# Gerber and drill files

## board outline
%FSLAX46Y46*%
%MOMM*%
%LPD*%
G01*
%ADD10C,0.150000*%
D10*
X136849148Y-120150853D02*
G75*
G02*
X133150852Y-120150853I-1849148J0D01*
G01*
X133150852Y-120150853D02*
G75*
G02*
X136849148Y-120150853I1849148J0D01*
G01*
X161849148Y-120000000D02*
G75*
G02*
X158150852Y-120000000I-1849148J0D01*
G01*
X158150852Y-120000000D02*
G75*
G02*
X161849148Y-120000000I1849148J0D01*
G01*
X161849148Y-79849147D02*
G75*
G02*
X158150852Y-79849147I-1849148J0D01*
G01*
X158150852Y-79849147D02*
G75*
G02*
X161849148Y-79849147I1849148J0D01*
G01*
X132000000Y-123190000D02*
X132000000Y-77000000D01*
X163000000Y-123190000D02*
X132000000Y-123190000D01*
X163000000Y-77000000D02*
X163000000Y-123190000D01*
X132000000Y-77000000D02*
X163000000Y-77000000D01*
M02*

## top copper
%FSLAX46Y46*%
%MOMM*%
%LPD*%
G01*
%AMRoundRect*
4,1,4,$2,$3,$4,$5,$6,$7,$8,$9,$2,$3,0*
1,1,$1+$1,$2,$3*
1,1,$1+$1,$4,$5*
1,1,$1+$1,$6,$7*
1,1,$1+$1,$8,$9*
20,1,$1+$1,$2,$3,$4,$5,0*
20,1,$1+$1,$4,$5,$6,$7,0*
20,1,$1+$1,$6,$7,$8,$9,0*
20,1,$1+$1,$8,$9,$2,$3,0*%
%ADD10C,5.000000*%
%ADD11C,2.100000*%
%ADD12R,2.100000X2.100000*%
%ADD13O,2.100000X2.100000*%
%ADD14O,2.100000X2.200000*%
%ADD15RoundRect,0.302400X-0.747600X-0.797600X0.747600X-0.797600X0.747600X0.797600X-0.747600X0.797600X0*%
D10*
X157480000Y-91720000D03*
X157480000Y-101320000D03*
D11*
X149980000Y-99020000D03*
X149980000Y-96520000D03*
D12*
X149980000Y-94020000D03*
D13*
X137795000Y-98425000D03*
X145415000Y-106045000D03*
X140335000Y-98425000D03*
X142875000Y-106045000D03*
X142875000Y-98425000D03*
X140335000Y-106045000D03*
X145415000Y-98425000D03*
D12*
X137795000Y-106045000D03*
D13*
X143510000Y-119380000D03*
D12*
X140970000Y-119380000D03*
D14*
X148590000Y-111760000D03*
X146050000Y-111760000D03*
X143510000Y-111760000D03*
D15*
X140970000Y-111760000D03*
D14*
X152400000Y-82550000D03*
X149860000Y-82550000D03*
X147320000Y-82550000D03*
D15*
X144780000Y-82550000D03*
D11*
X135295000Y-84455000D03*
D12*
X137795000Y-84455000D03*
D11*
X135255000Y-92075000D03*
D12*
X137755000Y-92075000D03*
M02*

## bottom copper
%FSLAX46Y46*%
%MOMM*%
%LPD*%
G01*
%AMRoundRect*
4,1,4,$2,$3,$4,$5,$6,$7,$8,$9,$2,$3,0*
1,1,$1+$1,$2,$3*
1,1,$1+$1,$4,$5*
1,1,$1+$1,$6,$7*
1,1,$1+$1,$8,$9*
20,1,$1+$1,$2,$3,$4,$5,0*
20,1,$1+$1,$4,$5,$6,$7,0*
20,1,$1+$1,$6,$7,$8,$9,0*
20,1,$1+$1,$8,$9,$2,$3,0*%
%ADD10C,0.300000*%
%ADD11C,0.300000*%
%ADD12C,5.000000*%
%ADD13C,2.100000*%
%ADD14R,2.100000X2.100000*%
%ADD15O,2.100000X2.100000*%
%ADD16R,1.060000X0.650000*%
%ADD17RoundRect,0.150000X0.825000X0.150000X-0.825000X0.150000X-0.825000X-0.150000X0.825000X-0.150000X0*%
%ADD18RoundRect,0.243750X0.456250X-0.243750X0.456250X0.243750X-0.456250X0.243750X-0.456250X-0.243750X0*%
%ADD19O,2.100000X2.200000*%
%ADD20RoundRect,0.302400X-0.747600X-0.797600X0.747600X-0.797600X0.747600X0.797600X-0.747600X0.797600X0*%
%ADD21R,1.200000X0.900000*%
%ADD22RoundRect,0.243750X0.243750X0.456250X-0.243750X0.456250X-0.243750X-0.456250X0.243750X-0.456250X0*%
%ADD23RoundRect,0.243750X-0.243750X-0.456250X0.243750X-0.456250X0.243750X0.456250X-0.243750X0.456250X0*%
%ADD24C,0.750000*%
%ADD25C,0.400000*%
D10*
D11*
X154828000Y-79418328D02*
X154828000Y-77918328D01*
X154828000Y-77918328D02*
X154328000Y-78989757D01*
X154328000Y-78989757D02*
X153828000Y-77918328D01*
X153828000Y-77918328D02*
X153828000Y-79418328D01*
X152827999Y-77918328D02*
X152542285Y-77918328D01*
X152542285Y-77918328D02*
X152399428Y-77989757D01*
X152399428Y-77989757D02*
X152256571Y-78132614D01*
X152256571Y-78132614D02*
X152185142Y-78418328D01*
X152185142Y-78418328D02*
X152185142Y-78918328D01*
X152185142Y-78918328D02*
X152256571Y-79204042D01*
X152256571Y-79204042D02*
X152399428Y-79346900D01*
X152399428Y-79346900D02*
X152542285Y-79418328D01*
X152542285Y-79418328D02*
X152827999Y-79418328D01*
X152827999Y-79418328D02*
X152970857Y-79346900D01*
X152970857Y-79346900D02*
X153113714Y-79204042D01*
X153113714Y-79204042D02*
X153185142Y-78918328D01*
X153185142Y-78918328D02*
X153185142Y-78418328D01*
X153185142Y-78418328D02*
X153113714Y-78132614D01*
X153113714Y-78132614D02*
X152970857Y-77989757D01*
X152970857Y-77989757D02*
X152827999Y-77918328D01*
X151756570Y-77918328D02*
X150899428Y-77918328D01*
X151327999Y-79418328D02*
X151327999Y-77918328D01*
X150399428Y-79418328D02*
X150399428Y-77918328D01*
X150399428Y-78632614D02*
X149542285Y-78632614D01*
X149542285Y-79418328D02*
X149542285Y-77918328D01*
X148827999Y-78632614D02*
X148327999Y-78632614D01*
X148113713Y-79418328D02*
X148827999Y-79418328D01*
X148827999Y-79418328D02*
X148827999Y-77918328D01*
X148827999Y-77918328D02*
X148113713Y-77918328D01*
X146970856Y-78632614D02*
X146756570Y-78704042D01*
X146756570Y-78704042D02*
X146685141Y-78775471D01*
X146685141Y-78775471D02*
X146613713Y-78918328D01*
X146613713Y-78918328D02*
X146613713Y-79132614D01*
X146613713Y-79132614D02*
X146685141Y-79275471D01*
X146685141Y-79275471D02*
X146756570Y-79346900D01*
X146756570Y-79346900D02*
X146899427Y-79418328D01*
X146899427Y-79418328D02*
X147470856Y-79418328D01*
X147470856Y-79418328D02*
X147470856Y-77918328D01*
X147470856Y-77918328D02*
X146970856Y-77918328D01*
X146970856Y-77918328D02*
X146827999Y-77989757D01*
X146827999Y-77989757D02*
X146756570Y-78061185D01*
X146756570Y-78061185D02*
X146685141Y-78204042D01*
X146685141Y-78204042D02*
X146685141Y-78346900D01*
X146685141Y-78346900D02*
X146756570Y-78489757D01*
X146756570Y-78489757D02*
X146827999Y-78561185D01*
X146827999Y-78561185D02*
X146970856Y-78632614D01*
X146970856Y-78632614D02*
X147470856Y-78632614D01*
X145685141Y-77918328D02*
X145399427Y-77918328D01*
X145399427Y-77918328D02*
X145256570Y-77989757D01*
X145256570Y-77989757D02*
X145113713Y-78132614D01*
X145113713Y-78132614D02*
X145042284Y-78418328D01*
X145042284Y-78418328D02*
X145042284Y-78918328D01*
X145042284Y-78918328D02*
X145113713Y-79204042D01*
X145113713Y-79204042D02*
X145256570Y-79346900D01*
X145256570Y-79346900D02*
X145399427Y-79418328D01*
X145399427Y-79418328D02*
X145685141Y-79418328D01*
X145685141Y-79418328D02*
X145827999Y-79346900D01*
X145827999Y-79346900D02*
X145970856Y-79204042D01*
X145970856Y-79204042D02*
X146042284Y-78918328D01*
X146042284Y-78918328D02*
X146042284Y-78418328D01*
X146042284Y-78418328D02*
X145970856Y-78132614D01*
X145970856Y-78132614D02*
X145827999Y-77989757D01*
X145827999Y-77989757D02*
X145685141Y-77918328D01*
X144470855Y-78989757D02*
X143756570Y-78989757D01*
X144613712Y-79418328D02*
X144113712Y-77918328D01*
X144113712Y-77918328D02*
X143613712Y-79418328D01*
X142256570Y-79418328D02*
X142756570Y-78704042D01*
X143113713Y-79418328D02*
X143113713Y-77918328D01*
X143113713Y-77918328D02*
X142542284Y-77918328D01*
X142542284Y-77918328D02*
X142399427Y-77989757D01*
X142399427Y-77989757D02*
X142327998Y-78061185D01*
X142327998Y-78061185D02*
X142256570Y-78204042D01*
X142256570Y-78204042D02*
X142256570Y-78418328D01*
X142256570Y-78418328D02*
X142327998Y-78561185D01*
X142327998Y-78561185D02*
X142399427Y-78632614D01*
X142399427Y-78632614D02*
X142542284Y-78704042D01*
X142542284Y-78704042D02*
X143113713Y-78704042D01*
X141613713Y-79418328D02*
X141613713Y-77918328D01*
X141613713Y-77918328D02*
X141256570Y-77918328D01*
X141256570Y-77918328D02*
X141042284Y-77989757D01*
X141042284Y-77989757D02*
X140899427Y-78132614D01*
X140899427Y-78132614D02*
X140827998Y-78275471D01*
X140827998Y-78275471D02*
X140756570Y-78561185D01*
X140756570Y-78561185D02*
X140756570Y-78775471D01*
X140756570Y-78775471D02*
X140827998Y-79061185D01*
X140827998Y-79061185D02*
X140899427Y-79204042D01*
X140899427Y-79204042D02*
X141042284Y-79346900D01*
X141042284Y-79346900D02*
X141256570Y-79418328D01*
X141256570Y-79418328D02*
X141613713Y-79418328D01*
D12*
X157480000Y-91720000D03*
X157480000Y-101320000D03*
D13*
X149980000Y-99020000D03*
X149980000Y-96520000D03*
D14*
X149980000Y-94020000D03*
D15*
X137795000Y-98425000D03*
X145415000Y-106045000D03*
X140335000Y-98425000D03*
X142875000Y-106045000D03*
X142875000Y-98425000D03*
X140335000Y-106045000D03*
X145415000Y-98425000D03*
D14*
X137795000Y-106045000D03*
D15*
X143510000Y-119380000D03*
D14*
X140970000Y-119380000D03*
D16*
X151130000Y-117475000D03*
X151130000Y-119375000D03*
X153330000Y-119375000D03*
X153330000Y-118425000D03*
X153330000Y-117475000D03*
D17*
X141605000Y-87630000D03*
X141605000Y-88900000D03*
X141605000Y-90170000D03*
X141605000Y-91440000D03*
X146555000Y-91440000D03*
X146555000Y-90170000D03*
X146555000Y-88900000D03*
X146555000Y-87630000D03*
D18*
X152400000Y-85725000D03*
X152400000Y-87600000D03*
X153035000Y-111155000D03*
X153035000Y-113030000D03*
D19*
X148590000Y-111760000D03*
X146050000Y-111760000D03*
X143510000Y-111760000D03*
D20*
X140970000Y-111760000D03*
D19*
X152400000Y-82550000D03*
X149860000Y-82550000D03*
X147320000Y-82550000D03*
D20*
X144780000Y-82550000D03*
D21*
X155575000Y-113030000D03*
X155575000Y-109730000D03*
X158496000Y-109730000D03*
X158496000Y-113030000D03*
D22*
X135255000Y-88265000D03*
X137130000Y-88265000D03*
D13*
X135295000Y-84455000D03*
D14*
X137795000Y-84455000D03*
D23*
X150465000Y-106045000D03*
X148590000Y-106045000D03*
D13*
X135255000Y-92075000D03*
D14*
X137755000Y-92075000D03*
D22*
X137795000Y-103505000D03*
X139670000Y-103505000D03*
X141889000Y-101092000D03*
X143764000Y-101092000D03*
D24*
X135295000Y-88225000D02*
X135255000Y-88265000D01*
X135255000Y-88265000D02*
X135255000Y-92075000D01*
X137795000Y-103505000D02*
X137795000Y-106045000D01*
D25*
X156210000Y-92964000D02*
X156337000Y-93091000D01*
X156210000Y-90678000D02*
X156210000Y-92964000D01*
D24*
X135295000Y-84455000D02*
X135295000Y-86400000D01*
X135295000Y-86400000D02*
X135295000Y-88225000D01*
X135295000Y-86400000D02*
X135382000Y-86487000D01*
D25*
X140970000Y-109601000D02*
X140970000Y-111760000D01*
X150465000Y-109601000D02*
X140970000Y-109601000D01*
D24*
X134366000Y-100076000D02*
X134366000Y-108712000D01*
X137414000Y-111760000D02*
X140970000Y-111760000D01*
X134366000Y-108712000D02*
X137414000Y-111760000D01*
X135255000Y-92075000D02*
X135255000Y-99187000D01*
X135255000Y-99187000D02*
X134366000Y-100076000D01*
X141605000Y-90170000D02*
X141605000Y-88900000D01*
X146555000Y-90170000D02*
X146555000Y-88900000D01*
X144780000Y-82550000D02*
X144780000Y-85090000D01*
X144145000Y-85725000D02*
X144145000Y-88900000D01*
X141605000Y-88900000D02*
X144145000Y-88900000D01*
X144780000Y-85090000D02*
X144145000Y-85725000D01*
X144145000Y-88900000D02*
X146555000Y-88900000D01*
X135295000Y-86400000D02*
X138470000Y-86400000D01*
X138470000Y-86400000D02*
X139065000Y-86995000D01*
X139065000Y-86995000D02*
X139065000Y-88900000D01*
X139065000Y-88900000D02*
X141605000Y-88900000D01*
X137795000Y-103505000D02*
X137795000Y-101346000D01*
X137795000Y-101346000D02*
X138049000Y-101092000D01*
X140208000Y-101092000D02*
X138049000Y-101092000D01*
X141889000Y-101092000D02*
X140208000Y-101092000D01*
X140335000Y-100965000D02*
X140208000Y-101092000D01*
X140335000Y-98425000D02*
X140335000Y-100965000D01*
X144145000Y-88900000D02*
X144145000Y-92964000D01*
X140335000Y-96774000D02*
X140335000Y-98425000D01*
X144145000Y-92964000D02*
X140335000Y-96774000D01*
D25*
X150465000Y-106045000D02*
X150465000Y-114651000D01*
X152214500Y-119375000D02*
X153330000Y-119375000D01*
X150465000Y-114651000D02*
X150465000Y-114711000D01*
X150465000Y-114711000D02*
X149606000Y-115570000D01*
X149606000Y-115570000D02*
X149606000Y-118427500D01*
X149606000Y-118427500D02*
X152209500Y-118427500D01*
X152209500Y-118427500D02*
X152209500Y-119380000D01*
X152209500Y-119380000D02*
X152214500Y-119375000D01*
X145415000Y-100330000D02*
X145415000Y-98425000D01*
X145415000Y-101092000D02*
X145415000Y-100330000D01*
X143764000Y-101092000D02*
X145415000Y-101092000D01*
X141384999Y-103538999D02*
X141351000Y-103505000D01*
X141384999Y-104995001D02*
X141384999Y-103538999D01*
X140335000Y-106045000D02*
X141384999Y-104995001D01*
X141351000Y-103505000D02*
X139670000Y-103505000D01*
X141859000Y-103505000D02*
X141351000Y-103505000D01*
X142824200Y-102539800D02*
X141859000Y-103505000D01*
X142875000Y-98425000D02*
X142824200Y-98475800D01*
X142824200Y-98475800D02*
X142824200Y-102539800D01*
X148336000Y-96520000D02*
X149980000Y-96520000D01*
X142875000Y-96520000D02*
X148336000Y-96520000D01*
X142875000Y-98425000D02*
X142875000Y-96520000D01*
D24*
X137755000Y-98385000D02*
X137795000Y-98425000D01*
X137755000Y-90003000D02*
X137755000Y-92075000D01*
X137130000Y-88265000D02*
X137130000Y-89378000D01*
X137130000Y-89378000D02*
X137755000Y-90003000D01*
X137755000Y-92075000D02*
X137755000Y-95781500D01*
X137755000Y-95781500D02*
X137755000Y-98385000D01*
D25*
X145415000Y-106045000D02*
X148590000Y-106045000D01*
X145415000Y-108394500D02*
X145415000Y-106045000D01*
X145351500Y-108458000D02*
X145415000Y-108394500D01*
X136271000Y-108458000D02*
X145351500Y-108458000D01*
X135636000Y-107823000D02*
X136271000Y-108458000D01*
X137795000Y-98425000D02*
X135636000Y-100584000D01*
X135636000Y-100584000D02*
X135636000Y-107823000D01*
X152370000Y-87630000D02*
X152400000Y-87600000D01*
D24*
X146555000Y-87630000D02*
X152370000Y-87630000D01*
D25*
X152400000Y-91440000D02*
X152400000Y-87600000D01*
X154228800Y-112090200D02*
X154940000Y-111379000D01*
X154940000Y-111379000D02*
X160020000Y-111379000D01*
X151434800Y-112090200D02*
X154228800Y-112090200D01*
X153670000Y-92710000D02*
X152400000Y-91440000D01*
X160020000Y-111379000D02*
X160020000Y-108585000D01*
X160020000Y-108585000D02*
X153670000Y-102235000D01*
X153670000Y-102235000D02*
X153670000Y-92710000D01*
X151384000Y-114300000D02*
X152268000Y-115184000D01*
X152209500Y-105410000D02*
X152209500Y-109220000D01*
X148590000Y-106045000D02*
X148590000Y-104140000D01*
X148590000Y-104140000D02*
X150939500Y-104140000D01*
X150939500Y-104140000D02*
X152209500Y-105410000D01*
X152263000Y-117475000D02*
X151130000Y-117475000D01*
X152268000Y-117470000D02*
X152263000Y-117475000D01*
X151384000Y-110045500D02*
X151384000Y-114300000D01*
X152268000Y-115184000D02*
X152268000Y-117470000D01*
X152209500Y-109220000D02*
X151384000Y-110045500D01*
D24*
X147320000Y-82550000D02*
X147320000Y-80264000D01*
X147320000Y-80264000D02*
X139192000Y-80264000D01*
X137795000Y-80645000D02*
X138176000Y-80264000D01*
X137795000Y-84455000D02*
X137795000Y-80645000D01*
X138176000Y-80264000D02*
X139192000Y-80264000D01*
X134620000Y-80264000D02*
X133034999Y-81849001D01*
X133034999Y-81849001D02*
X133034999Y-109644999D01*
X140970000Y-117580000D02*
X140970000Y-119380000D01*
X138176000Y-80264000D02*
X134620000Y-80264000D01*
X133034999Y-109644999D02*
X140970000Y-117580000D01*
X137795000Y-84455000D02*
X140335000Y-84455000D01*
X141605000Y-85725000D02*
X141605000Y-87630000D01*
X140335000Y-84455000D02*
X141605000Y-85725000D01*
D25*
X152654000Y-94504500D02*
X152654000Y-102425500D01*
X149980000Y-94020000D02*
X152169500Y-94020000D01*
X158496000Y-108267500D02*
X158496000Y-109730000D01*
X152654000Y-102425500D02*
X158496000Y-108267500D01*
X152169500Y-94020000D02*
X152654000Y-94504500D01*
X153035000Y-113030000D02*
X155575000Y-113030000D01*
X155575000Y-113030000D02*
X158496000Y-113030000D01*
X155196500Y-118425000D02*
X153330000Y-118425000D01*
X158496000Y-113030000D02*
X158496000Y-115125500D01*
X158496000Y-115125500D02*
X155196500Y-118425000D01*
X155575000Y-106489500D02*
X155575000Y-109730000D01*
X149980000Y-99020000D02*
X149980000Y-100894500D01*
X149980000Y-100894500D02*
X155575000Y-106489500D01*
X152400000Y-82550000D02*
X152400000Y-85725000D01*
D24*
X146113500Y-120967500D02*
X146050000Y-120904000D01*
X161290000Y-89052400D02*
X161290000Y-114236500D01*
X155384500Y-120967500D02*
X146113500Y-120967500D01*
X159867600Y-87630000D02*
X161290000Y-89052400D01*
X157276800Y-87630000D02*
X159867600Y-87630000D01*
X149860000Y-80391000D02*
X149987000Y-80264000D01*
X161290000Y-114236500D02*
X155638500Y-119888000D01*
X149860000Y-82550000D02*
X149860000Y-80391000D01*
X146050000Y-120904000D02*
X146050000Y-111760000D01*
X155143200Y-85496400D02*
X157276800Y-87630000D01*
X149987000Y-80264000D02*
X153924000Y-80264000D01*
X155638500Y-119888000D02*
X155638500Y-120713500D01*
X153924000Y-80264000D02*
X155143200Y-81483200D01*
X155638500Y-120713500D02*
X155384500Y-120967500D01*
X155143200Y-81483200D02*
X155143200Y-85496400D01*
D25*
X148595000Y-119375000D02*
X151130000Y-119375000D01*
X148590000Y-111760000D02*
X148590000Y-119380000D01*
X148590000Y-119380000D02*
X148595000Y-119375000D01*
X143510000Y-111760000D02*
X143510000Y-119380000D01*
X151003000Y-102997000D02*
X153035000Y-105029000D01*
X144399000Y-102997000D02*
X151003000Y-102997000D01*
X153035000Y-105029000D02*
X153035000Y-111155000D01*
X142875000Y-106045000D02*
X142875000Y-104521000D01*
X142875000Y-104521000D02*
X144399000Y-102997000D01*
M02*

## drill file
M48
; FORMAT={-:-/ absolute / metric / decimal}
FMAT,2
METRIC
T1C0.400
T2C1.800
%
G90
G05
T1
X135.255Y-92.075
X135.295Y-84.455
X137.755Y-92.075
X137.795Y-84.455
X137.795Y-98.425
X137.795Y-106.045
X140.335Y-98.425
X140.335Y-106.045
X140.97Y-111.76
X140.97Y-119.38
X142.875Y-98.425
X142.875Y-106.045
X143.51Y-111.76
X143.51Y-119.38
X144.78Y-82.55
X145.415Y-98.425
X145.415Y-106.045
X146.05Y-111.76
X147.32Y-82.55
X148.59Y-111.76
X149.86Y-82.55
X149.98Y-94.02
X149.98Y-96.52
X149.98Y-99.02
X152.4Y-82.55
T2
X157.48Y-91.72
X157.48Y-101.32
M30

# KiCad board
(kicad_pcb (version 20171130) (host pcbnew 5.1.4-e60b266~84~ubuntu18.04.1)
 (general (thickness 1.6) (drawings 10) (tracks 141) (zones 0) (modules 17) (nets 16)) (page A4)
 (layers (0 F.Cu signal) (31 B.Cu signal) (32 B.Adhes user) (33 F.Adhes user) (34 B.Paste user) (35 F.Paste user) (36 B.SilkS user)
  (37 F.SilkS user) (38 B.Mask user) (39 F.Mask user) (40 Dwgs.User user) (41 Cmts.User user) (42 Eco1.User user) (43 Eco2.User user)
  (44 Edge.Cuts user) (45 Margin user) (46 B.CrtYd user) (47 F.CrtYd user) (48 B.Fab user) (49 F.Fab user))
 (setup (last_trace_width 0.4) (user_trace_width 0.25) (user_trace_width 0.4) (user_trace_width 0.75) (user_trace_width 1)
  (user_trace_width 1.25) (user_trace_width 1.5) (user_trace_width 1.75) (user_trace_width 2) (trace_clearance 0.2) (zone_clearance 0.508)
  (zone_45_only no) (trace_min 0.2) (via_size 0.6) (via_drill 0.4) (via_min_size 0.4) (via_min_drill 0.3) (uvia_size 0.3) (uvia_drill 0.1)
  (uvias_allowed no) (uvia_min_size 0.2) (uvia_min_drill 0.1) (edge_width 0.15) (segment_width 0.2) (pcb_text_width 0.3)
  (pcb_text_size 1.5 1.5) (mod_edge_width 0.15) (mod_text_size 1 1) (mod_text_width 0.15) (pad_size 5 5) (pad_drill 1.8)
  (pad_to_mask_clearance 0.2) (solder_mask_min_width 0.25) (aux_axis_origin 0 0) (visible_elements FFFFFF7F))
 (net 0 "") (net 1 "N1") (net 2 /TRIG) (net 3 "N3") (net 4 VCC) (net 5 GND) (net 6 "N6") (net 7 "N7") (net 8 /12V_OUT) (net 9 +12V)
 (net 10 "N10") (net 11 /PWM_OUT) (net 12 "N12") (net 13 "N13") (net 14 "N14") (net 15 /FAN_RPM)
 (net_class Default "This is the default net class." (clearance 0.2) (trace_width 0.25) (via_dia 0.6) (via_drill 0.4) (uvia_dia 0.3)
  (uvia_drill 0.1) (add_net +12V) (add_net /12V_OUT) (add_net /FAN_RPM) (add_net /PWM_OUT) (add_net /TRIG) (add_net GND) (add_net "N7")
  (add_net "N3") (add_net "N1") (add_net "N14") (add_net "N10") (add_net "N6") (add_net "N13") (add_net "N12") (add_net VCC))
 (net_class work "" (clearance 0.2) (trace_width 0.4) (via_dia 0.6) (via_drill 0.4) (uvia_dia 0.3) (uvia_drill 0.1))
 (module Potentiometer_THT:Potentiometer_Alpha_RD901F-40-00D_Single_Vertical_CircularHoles (layer F.Cu) (at 149.98 94.02)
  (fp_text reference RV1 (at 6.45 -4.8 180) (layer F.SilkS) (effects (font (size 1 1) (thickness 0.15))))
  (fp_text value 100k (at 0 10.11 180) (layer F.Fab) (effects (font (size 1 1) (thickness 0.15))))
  (pad "" thru_hole circle (at 7.5 -2.3 90) (size 5 5) (drill 1.8) (layers *.Cu *.Mask))
  (pad "" thru_hole circle (at 7.5 7.3 90) (size 5 5) (drill 1.8) (layers *.Cu *.Mask))
  (pad 3 thru_hole circle (at 0 5 90) (size 2.1 2.1) (drill 0.4) (layers *.Cu *.Mask) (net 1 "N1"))
  (pad 2 thru_hole circle (at 0 2.5 90) (size 2.1 2.1) (drill 0.4) (layers *.Cu *.Mask) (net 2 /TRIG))
  (pad 1 thru_hole rect (at 0 0 90) (size 2.1 2.1) (drill 0.4) (layers *.Cu *.Mask) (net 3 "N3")))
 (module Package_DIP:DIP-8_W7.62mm (layer F.Cu) (at 137.795 106.045 90)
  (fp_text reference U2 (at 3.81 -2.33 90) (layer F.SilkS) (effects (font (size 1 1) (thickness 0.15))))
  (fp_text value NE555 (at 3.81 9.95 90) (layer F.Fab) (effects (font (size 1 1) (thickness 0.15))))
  (pad 8 thru_hole oval (at 7.62 0 90) (size 2.1 2.1) (drill 0.4) (layers *.Cu *.Mask) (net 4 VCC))
  (pad 4 thru_hole oval (at 0 7.62 90) (size 2.1 2.1) (drill 0.4) (layers *.Cu *.Mask) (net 4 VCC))
  (pad 7 thru_hole oval (at 7.62 2.54 90) (size 2.1 2.1) (drill 0.4) (layers *.Cu *.Mask) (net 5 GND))
  (pad 3 thru_hole oval (at 0 5.08 90) (size 2.1 2.1) (drill 0.4) (layers *.Cu *.Mask) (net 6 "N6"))
  (pad 6 thru_hole oval (at 7.62 5.08 90) (size 2.1 2.1) (drill 0.4) (layers *.Cu *.Mask) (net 2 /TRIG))
  (pad 2 thru_hole oval (at 0 2.54 90) (size 2.1 2.1) (drill 0.4) (layers *.Cu *.Mask) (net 2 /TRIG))
  (pad 5 thru_hole oval (at 7.62 7.62 90) (size 2.1 2.1) (drill 0.4) (layers *.Cu *.Mask) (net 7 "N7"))
  (pad 1 thru_hole rect (at 0 0 90) (size 2.1 2.1) (drill 0.4) (layers *.Cu *.Mask) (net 5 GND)))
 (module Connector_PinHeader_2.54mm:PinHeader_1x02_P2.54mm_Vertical (layer F.Cu) (at 140.97 119.38 90)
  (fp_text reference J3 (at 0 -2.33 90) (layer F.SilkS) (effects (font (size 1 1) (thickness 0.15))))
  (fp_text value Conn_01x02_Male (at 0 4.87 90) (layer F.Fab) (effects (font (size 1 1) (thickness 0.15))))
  (pad 2 thru_hole oval (at 0 2.54 90) (size 2.1 2.1) (drill 0.4) (layers *.Cu *.Mask) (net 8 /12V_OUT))
  (pad 1 thru_hole rect (at 0 0 90) (size 2.1 2.1) (drill 0.4) (layers *.Cu *.Mask) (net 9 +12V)))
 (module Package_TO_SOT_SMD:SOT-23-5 (layer B.Cu) (at 152.23 118.425 180)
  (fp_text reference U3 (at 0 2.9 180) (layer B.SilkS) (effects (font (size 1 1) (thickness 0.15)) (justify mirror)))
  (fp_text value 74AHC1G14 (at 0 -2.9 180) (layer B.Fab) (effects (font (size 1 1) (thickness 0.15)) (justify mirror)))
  (pad 5 smd rect (at 1.1 0.95 180) (size 1.06 0.65) (layers B.Cu B.Paste B.Mask) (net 4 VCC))
  (pad 4 smd rect (at 1.1 -0.95 180) (size 1.06 0.65) (layers B.Cu B.Paste B.Mask) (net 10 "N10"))
  (pad 3 smd rect (at -1.1 -0.95 180) (size 1.06 0.65) (layers B.Cu B.Paste B.Mask) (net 5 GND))
  (pad 2 smd rect (at -1.1 0 180) (size 1.06 0.65) (layers B.Cu B.Paste B.Mask) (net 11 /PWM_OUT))
  (pad 1 smd rect (at -1.1 0.95 180) (size 1.06 0.65) (layers B.Cu B.Paste B.Mask)))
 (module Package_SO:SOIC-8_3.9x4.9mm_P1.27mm (layer B.Cu) (at 144.08 89.535 180)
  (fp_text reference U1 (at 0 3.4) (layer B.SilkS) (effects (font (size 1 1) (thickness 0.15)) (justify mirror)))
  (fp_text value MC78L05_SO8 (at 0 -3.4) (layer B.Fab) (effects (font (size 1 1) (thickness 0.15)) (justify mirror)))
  (pad 8 smd roundrect (at 2.475 1.905 180) (size 1.95 0.6) (layers B.Cu B.Paste B.Mask) (roundrect_rratio 0.25) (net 9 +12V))
  (pad 7 smd roundrect (at 2.475 0.635 180) (size 1.95 0.6) (layers B.Cu B.Paste B.Mask) (roundrect_rratio 0.25) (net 5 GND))
  (pad 6 smd roundrect (at 2.475 -0.635 180) (size 1.95 0.6) (layers B.Cu B.Paste B.Mask) (roundrect_rratio 0.25) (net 5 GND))
  (pad 5 smd roundrect (at 2.475 -1.905 180) (size 1.95 0.6) (layers B.Cu B.Paste B.Mask) (roundrect_rratio 0.25) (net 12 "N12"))
  (pad 4 smd roundrect (at -2.475 -1.905 180) (size 1.95 0.6) (layers B.Cu B.Paste B.Mask) (roundrect_rratio 0.25) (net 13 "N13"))
  (pad 3 smd roundrect (at -2.475 -0.635 180) (size 1.95 0.6) (layers B.Cu B.Paste B.Mask) (roundrect_rratio 0.25) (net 5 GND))
  (pad 2 smd roundrect (at -2.475 0.635 180) (size 1.95 0.6) (layers B.Cu B.Paste B.Mask) (roundrect_rratio 0.25) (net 5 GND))
  (pad 1 smd roundrect (at -2.475 1.905 180) (size 1.95 0.6) (layers B.Cu B.Paste B.Mask) (roundrect_rratio 0.25) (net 4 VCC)))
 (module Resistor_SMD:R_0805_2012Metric (layer B.Cu) (at 152.4 86.6625 90)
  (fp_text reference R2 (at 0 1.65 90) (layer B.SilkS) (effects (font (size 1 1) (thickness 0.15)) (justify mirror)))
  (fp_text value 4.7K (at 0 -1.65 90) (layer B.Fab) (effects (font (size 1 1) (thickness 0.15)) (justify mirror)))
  (pad 2 smd roundrect (at 0.9375 0 90) (size 0.975 1.4) (layers B.Cu B.Paste B.Mask) (roundrect_rratio 0.25) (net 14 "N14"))
  (pad 1 smd roundrect (at -0.9375 0 90) (size 0.975 1.4) (layers B.Cu B.Paste B.Mask) (roundrect_rratio 0.25) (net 4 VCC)))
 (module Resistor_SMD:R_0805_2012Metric (layer B.Cu) (at 153.035 112.0925 90)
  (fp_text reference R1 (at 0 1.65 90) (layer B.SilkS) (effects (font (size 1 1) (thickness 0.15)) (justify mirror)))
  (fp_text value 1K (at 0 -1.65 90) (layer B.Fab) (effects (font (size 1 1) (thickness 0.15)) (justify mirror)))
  (pad 2 smd roundrect (at 0.9375 0 90) (size 0.975 1.4) (layers B.Cu B.Paste B.Mask) (roundrect_rratio 0.25) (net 6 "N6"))
  (pad 1 smd roundrect (at -0.9375 0 90) (size 0.975 1.4) (layers B.Cu B.Paste B.Mask) (roundrect_rratio 0.25) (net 11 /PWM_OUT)))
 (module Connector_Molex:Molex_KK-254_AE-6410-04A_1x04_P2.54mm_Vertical (layer F.Cu) (at 140.97 111.76)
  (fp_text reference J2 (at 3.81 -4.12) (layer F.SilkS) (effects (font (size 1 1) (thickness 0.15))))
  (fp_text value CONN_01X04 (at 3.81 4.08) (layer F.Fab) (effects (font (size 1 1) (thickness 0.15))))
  (pad 4 thru_hole oval (at 7.62 0) (size 2.1 2.2) (drill 0.4) (layers *.Cu *.Mask) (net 10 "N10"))
  (pad 3 thru_hole oval (at 5.08 0) (size 2.1 2.2) (drill 0.4) (layers *.Cu *.Mask) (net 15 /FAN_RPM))
  (pad 2 thru_hole oval (at 2.54 0) (size 2.1 2.2) (drill 0.4) (layers *.Cu *.Mask) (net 8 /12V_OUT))
  (pad 1 thru_hole roundrect (at 0 0) (size 2.1 2.2) (drill 0.4) (layers *.Cu *.Mask) (roundrect_rratio 0.144) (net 5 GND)))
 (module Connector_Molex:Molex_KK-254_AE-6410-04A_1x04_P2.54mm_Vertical (layer F.Cu) (at 144.78 82.55)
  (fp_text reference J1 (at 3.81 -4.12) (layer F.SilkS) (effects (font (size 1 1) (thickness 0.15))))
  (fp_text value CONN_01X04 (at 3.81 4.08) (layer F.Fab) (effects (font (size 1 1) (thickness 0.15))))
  (pad 4 thru_hole oval (at 7.62 0) (size 2.1 2.2) (drill 0.4) (layers *.Cu *.Mask) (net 14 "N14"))
  (pad 3 thru_hole oval (at 5.08 0) (size 2.1 2.2) (drill 0.4) (layers *.Cu *.Mask) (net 15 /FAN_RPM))
  (pad 2 thru_hole oval (at 2.54 0) (size 2.1 2.2) (drill 0.4) (layers *.Cu *.Mask) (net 9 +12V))
  (pad 1 thru_hole roundrect (at 0 0) (size 2.1 2.2) (drill 0.4) (layers *.Cu *.Mask) (roundrect_rratio 0.144) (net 5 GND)))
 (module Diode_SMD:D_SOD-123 (layer B.Cu) (at 155.575 111.38 270)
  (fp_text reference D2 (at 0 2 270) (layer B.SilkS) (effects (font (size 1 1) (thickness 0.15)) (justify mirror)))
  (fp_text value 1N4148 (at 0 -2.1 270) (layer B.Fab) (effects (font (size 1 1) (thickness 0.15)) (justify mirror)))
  (pad 2 smd rect (at 1.65 0 270) (size 0.9 1.2) (layers B.Cu B.Paste B.Mask) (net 11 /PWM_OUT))
  (pad 1 smd rect (at -1.65 0 270) (size 0.9 1.2) (layers B.Cu B.Paste B.Mask) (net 1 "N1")))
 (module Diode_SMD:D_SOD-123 (layer B.Cu) (at 158.496 111.38 90)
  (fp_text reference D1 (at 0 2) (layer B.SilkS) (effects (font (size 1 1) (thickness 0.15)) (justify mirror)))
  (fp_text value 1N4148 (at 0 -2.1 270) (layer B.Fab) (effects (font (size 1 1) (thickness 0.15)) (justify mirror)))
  (pad 2 smd rect (at 1.65 0 90) (size 0.9 1.2) (layers B.Cu B.Paste B.Mask) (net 3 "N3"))
  (pad 1 smd rect (at -1.65 0 90) (size 0.9 1.2) (layers B.Cu B.Paste B.Mask) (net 11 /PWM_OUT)))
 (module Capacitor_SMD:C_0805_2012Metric (layer B.Cu) (at 136.1925 88.265 180)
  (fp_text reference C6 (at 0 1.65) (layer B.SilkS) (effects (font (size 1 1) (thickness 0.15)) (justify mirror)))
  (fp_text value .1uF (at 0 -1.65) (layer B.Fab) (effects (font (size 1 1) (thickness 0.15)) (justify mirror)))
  (pad 2 smd roundrect (at 0.9375 0 180) (size 0.975 1.4) (layers B.Cu B.Paste B.Mask) (roundrect_rratio 0.25) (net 5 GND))
  (pad 1 smd roundrect (at -0.9375 0 180) (size 0.975 1.4) (layers B.Cu B.Paste B.Mask) (roundrect_rratio 0.25) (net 4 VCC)))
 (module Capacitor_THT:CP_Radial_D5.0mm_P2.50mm (layer F.Cu) (at 137.795 84.455 180)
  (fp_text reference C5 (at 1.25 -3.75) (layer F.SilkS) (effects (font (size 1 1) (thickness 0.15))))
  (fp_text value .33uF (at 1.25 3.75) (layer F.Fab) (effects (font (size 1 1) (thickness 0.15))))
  (pad 2 thru_hole circle (at 2.5 0 180) (size 2.1 2.1) (drill 0.4) (layers *.Cu *.Mask) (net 5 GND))
  (pad 1 thru_hole rect (at 0 0 180) (size 2.1 2.1) (drill 0.4) (layers *.Cu *.Mask) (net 9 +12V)))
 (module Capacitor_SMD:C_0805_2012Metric (layer B.Cu) (at 149.5275 106.045)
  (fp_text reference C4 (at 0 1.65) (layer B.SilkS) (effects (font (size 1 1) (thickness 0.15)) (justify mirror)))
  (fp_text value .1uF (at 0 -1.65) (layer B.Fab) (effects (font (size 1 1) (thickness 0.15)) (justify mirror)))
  (pad 2 smd roundrect (at 0.9375 0) (size 0.975 1.4) (layers B.Cu B.Paste B.Mask) (roundrect_rratio 0.25) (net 5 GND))
  (pad 1 smd roundrect (at -0.9375 0) (size 0.975 1.4) (layers B.Cu B.Paste B.Mask) (roundrect_rratio 0.25) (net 4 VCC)))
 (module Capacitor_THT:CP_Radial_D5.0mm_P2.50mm (layer F.Cu) (at 137.755 92.075 180)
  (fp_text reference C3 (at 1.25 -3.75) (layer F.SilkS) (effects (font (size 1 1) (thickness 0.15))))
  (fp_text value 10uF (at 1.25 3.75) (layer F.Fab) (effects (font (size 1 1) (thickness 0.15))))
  (pad 2 thru_hole circle (at 2.5 0 180) (size 2.1 2.1) (drill 0.4) (layers *.Cu *.Mask) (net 5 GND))
  (pad 1 thru_hole rect (at 0 0 180) (size 2.1 2.1) (drill 0.4) (layers *.Cu *.Mask) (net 4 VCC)))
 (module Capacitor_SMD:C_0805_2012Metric (layer B.Cu) (at 138.7325 103.505 180)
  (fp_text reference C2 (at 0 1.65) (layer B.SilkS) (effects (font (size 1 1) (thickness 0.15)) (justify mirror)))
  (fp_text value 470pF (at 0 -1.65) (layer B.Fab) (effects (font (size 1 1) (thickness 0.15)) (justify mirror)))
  (pad 2 smd roundrect (at 0.9375 0 180) (size 0.975 1.4) (layers B.Cu B.Paste B.Mask) (roundrect_rratio 0.25) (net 5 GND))
  (pad 1 smd roundrect (at -0.9375 0 180) (size 0.975 1.4) (layers B.Cu B.Paste B.Mask) (roundrect_rratio 0.25) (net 2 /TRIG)))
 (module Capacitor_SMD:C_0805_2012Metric (layer B.Cu) (at 142.8265 101.092 180)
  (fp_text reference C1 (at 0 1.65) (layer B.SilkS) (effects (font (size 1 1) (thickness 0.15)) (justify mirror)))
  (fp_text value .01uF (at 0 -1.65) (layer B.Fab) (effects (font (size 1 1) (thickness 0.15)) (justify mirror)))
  (pad 2 smd roundrect (at 0.9375 0 180) (size 0.975 1.4) (layers B.Cu B.Paste B.Mask) (roundrect_rratio 0.25) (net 5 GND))
  (pad 1 smd roundrect (at -0.9375 0 180) (size 0.975 1.4) (layers B.Cu B.Paste B.Mask) (roundrect_rratio 0.25) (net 7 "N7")))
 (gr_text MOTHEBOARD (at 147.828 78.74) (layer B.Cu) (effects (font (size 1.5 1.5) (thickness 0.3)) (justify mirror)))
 (gr_circle (center 135 120.150853) (end 136.778 120.658853) (layer Edge.Cuts) (width 0.15))
 (gr_circle (center 160 120) (end 161.778 120.508) (layer Edge.Cuts) (width 0.15))
 (gr_circle (center 160 79.849147) (end 161.778 80.357147) (layer Edge.Cuts) (width 0.15))
 (gr_line (start 132 123.19) (end 132 77) (layer Edge.Cuts) (width 0.15))
 (gr_line (start 163 123.19) (end 132 123.19) (layer Edge.Cuts) (width 0.15))
 (gr_line (start 163 77) (end 163 123.19) (layer Edge.Cuts) (width 0.15))
 (gr_line (start 132 77) (end 163 77) (layer Edge.Cuts) (width 0.15))
 (segment (start 135.295 88.225) (end 135.255 88.265) (width 0.75) (layer B.Cu) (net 5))
 (segment (start 135.255 88.265) (end 135.255 92.075) (width 0.75) (layer B.Cu) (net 5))
 (segment (start 137.795 103.505) (end 137.795 106.045) (width 0.75) (layer B.Cu) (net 5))
 (segment (start 156.21 92.964) (end 156.337 93.091) (width 0.4) (layer B.Cu) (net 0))
 (segment (start 156.21 90.678) (end 156.21 92.964) (width 0.4) (layer B.Cu) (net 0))
 (segment (start 135.295 84.455) (end 135.295 86.4) (width 0.75) (layer B.Cu) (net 5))
 (segment (start 135.295 86.4) (end 135.295 88.225) (width 0.75) (layer B.Cu) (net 5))
 (segment (start 135.295 86.4) (end 135.382 86.487) (width 0.75) (layer B.Cu) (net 5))
 (segment (start 140.97 109.601) (end 140.97 111.76) (width 0.4) (layer B.Cu) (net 5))
 (segment (start 150.465 109.601) (end 140.97 109.601) (width 0.4) (layer B.Cu) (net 5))
 (segment (start 134.366 100.076) (end 134.366 108.712) (width 0.75) (layer B.Cu) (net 5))
 (segment (start 137.414 111.76) (end 140.97 111.76) (width 0.75) (layer B.Cu) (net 5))
 (segment (start 134.366 108.712) (end 137.414 111.76) (width 0.75) (layer B.Cu) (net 5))
 (segment (start 135.255 92.075) (end 135.255 99.187) (width 0.75) (layer B.Cu) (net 5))
 (segment (start 135.255 99.187) (end 134.366 100.076) (width 0.75) (layer B.Cu) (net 5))
 (segment (start 141.605 90.17) (end 141.605 88.9) (width 0.75) (layer B.Cu) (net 5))
 (segment (start 146.555 90.17) (end 146.555 88.9) (width 0.75) (layer B.Cu) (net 5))
 (segment (start 144.78 82.55) (end 144.78 85.09) (width 0.75) (layer B.Cu) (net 5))
 (segment (start 144.145 85.725) (end 144.145 88.9) (width 0.75) (layer B.Cu) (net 5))
 (segment (start 141.605 88.9) (end 144.145 88.9) (width 0.75) (layer B.Cu) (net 5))
 (segment (start 144.78 85.09) (end 144.145 85.725) (width 0.75) (layer B.Cu) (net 5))
 (segment (start 144.145 88.9) (end 146.555 88.9) (width 0.75) (layer B.Cu) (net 5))
 (segment (start 135.295 86.4) (end 138.47 86.4) (width 0.75) (layer B.Cu) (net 5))
 (segment (start 138.47 86.4) (end 139.065 86.995) (width 0.75) (layer B.Cu) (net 5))
 (segment (start 139.065 86.995) (end 139.065 88.9) (width 0.75) (layer B.Cu) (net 5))
 (segment (start 139.065 88.9) (end 141.605 88.9) (width 0.75) (layer B.Cu) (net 5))
 (segment (start 137.795 103.505) (end 137.795 101.346) (width 0.75) (layer B.Cu) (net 5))
 (segment (start 137.795 101.346) (end 138.049 101.092) (width 0.75) (layer B.Cu) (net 5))
 (segment (start 140.208 101.092) (end 138.049 101.092) (width 0.75) (layer B.Cu) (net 5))
 (segment (start 141.889 101.092) (end 140.208 101.092) (width 0.75) (layer B.Cu) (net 5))
 (segment (start 140.335 100.965) (end 140.208 101.092) (width 0.75) (layer B.Cu) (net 5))
 (segment (start 140.335 98.425) (end 140.335 100.965) (width 0.75) (layer B.Cu) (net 5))
 (segment (start 144.145 88.9) (end 144.145 92.964) (width 0.75) (layer B.Cu) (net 5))
 (segment (start 140.335 96.774) (end 140.335 98.425) (width 0.75) (layer B.Cu) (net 5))
 (segment (start 144.145 92.964) (end 140.335 96.774) (width 0.75) (layer B.Cu) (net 5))
 (segment (start 150.465 106.045) (end 150.465 114.651) (width 0.4) (layer B.Cu) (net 5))
 (segment (start 152.2145 119.375) (end 153.33 119.375) (width 0.4) (layer B.Cu) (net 5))
 (segment (start 150.465 114.651) (end 150.465 114.711) (width 0.4) (layer B.Cu) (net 5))
 (segment (start 150.465 114.711) (end 149.606 115.57) (width 0.4) (layer B.Cu) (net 5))
 (segment (start 149.606 115.57) (end 149.606 118.4275) (width 0.4) (layer B.Cu) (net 5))
 (segment (start 149.606 118.4275) (end 152.2095 118.4275) (width 0.4) (layer B.Cu) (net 5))
 (segment (start 152.2095 118.4275) (end 152.2095 119.38) (width 0.4) (layer B.Cu) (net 5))
 (segment (start 152.2095 119.38) (end 152.2145 119.375) (width 0.4) (layer B.Cu) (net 5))
 (segment (start 145.415 100.33) (end 145.415 98.425) (width 0.4) (layer B.Cu) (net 7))
 (segment (start 145.415 101.092) (end 145.415 100.33) (width 0.4) (layer B.Cu) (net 7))
 (segment (start 143.764 101.092) (end 145.415 101.092) (width 0.4) (layer B.Cu) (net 7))
 (segment (start 141.384999 103.538999) (end 141.351 103.505) (width 0.4) (layer B.Cu) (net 2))
 (segment (start 141.384999 104.995001) (end 141.384999 103.538999) (width 0.4) (layer B.Cu) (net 2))
 (segment (start 140.335 106.045) (end 141.384999 104.995001) (width 0.4) (layer B.Cu) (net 2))
 (segment (start 141.351 103.505) (end 139.67 103.505) (width 0.4) (layer B.Cu) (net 2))
 (segment (start 141.859 103.505) (end 141.351 103.505) (width 0.4) (layer B.Cu) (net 2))
 (segment (start 142.8242 102.5398) (end 141.859 103.505) (width 0.4) (layer B.Cu) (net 2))
 (segment (start 142.875 98.425) (end 142.8242 98.4758) (width 0.4) (layer B.Cu) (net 2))
 (segment (start 142.8242 98.4758) (end 142.8242 102.5398) (width 0.4) (layer B.Cu) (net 2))
 (segment (start 148.336 96.52) (end 149.98 96.52) (width 0.4) (layer B.Cu) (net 2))
 (segment (start 142.875 96.52) (end 148.336 96.52) (width 0.4) (layer B.Cu) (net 2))
 (segment (start 142.875 98.425) (end 142.875 96.52) (width 0.4) (layer B.Cu) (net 2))
 (segment (start 137.755 98.385) (end 137.795 98.425) (width 0.75) (layer B.Cu) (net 4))
 (segment (start 137.755 90.003) (end 137.755 92.075) (width 0.75) (layer B.Cu) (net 4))
 (segment (start 137.13 88.265) (end 137.13 89.378) (width 0.75) (layer B.Cu) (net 4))
 (segment (start 137.13 89.378) (end 137.755 90.003) (width 0.75) (layer B.Cu) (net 4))
 (segment (start 137.755 92.075) (end 137.755 95.7815) (width 0.75) (layer B.Cu) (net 4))
 (segment (start 137.755 95.7815) (end 137.755 98.385) (width 0.75) (layer B.Cu) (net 4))
 (segment (start 145.415 106.045) (end 148.59 106.045) (width 0.4) (layer B.Cu) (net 4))
 (segment (start 145.415 108.3945) (end 145.415 106.045) (width 0.4) (layer B.Cu) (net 4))
 (segment (start 145.3515 108.458) (end 145.415 108.3945) (width 0.4) (layer B.Cu) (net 4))
 (segment (start 136.271 108.458) (end 145.3515 108.458) (width 0.4) (layer B.Cu) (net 4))
 (segment (start 135.636 107.823) (end 136.271 108.458) (width 0.4) (layer B.Cu) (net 4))
 (segment (start 137.795 98.425) (end 135.636 100.584) (width 0.4) (layer B.Cu) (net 4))
 (segment (start 135.636 100.584) (end 135.636 107.823) (width 0.4) (layer B.Cu) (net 4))
 (segment (start 152.37 87.63) (end 152.4 87.6) (width 0.4) (layer B.Cu) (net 4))
 (segment (start 146.555 87.63) (end 152.37 87.63) (width 0.75) (layer B.Cu) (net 4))
 (segment (start 152.4 91.44) (end 152.4 87.6) (width 0.4) (layer B.Cu) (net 4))
 (segment (start 154.2288 112.0902) (end 154.94 111.379) (width 0.4) (layer B.Cu) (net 4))
 (segment (start 154.94 111.379) (end 160.02 111.379) (width 0.4) (layer B.Cu) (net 4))
 (segment (start 151.4348 112.0902) (end 154.2288 112.0902) (width 0.4) (layer B.Cu) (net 4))
 (segment (start 153.67 92.71) (end 152.4 91.44) (width 0.4) (layer B.Cu) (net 4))
 (segment (start 160.02 111.379) (end 160.02 108.585) (width 0.4) (layer B.Cu) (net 4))
 (segment (start 160.02 108.585) (end 153.67 102.235) (width 0.4) (layer B.Cu) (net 4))
 (segment (start 153.67 102.235) (end 153.67 92.71) (width 0.4) (layer B.Cu) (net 4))
 (segment (start 151.384 114.3) (end 152.268 115.184) (width 0.4) (layer B.Cu) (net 4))
 (segment (start 152.2095 105.41) (end 152.2095 109.22) (width 0.4) (layer B.Cu) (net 4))
 (segment (start 148.59 106.045) (end 148.59 104.14) (width 0.4) (layer B.Cu) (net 4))
 (segment (start 148.59 104.14) (end 150.9395 104.14) (width 0.4) (layer B.Cu) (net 4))
 (segment (start 150.9395 104.14) (end 152.2095 105.41) (width 0.4) (layer B.Cu) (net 4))
 (segment (start 152.263 117.475) (end 151.13 117.475) (width 0.4) (layer B.Cu) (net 4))
 (segment (start 152.268 117.47) (end 152.263 117.475) (width 0.4) (layer B.Cu) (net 4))
 (segment (start 151.384 110.0455) (end 151.384 114.3) (width 0.4) (layer B.Cu) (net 4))
 (segment (start 152.268 115.184) (end 152.268 117.47) (width 0.4) (layer B.Cu) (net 4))
 (segment (start 152.2095 109.22) (end 151.384 110.0455) (width 0.4) (layer B.Cu) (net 4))
 (segment (start 147.32 82.55) (end 147.32 80.264) (width 0.75) (layer B.Cu) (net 9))
 (segment (start 147.32 80.264) (end 139.192 80.264) (width 0.75) (layer B.Cu) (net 9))
 (segment (start 137.795 80.645) (end 138.176 80.264) (width 0.75) (layer B.Cu) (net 9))
 (segment (start 137.795 84.455) (end 137.795 80.645) (width 0.75) (layer B.Cu) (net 9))
 (segment (start 138.176 80.264) (end 139.192 80.264) (width 0.75) (layer B.Cu) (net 9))
 (segment (start 134.62 80.264) (end 133.034999 81.849001) (width 0.75) (layer B.Cu) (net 9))
 (segment (start 133.034999 81.849001) (end 133.034999 109.644999) (width 0.75) (layer B.Cu) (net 9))
 (segment (start 140.97 117.58) (end 140.97 119.38) (width 0.75) (layer B.Cu) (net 9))
 (segment (start 138.176 80.264) (end 134.62 80.264) (width 0.75) (layer B.Cu) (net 9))
 (segment (start 133.034999 109.644999) (end 140.97 117.58) (width 0.75) (layer B.Cu) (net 9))
 (segment (start 137.795 84.455) (end 140.335 84.455) (width 0.75) (layer B.Cu) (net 9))
 (segment (start 141.605 85.725) (end 141.605 87.63) (width 0.75) (layer B.Cu) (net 9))
 (segment (start 140.335 84.455) (end 141.605 85.725) (width 0.75) (layer B.Cu) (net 9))
 (segment (start 152.654 94.5045) (end 152.654 102.4255) (width 0.4) (layer B.Cu) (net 3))
 (segment (start 149.98 94.02) (end 152.1695 94.02) (width 0.4) (layer B.Cu) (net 3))
 (segment (start 158.496 108.2675) (end 158.496 109.73) (width 0.4) (layer B.Cu) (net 3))
 (segment (start 152.654 102.4255) (end 158.496 108.2675) (width 0.4) (layer B.Cu) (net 3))
 (segment (start 152.1695 94.02) (end 152.654 94.5045) (width 0.4) (layer B.Cu) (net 3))
 (segment (start 153.035 113.03) (end 155.575 113.03) (width 0.4) (layer B.Cu) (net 11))
 (segment (start 155.575 113.03) (end 158.496 113.03) (width 0.4) (layer B.Cu) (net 11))
 (segment (start 155.1965 118.425) (end 153.33 118.425) (width 0.4) (layer B.Cu) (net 11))
 (segment (start 158.496 113.03) (end 158.496 115.1255) (width 0.4) (layer B.Cu) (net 11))
 (segment (start 158.496 115.1255) (end 155.1965 118.425) (width 0.4) (layer B.Cu) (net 11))
 (segment (start 155.575 106.4895) (end 155.575 109.73) (width 0.4) (layer B.Cu) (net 1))
 (segment (start 149.98 99.02) (end 149.98 100.8945) (width 0.4) (layer B.Cu) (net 1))
 (segment (start 149.98 100.8945) (end 155.575 106.4895) (width 0.4) (layer B.Cu) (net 1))
 (segment (start 152.4 82.55) (end 152.4 85.725) (width 0.4) (layer B.Cu) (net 14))
 (segment (start 146.1135 120.9675) (end 146.05 120.904) (width 0.75) (layer B.Cu) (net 15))
 (segment (start 161.29 89.0524) (end 161.29 114.2365) (width 0.75) (layer B.Cu) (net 15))
 (segment (start 155.3845 120.9675) (end 146.1135 120.9675) (width 0.75) (layer B.Cu) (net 15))
 (segment (start 159.8676 87.63) (end 161.29 89.0524) (width 0.75) (layer B.Cu) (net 15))
 (segment (start 157.2768 87.63) (end 159.8676 87.63) (width 0.75) (layer B.Cu) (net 15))
 (segment (start 149.86 80.391) (end 149.987 80.264) (width 0.75) (layer B.Cu) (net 15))
 (segment (start 161.29 114.2365) (end 155.6385 119.888) (width 0.75) (layer B.Cu) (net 15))
 (segment (start 149.86 82.55) (end 149.86 80.391) (width 0.75) (layer B.Cu) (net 15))
 (segment (start 146.05 120.904) (end 146.05 111.76) (width 0.75) (layer B.Cu) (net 15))
 (segment (start 155.1432 85.4964) (end 157.2768 87.63) (width 0.75) (layer B.Cu) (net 15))
 (segment (start 149.987 80.264) (end 153.924 80.264) (width 0.75) (layer B.Cu) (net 15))
 (segment (start 155.6385 119.888) (end 155.6385 120.7135) (width 0.75) (layer B.Cu) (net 15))
 (segment (start 153.924 80.264) (end 155.1432 81.4832) (width 0.75) (layer B.Cu) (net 15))
 (segment (start 155.6385 120.7135) (end 155.3845 120.9675) (width 0.75) (layer B.Cu) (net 15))
 (segment (start 155.1432 81.4832) (end 155.1432 85.4964) (width 0.75) (layer B.Cu) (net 15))
 (segment (start 148.595 119.375) (end 151.13 119.375) (width 0.4) (layer B.Cu) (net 10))
 (segment (start 148.59 111.76) (end 148.59 119.38) (width 0.4) (layer B.Cu) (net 10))
 (segment (start 148.59 119.38) (end 148.595 119.375) (width 0.4) (layer B.Cu) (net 10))
 (segment (start 143.51 111.76) (end 143.51 119.38) (width 0.4) (layer B.Cu) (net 8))
 (segment (start 151.003 102.997) (end 153.035 105.029) (width 0.4) (layer B.Cu) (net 6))
 (segment (start 144.399 102.997) (end 151.003 102.997) (width 0.4) (layer B.Cu) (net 6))
 (segment (start 153.035 105.029) (end 153.035 111.155) (width 0.4) (layer B.Cu) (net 6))
 (segment (start 142.875 106.045) (end 142.875 104.521) (width 0.4) (layer B.Cu) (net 6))
 (segment (start 142.875 104.521) (end 144.399 102.997) (width 0.4) (layer B.Cu) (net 6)))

